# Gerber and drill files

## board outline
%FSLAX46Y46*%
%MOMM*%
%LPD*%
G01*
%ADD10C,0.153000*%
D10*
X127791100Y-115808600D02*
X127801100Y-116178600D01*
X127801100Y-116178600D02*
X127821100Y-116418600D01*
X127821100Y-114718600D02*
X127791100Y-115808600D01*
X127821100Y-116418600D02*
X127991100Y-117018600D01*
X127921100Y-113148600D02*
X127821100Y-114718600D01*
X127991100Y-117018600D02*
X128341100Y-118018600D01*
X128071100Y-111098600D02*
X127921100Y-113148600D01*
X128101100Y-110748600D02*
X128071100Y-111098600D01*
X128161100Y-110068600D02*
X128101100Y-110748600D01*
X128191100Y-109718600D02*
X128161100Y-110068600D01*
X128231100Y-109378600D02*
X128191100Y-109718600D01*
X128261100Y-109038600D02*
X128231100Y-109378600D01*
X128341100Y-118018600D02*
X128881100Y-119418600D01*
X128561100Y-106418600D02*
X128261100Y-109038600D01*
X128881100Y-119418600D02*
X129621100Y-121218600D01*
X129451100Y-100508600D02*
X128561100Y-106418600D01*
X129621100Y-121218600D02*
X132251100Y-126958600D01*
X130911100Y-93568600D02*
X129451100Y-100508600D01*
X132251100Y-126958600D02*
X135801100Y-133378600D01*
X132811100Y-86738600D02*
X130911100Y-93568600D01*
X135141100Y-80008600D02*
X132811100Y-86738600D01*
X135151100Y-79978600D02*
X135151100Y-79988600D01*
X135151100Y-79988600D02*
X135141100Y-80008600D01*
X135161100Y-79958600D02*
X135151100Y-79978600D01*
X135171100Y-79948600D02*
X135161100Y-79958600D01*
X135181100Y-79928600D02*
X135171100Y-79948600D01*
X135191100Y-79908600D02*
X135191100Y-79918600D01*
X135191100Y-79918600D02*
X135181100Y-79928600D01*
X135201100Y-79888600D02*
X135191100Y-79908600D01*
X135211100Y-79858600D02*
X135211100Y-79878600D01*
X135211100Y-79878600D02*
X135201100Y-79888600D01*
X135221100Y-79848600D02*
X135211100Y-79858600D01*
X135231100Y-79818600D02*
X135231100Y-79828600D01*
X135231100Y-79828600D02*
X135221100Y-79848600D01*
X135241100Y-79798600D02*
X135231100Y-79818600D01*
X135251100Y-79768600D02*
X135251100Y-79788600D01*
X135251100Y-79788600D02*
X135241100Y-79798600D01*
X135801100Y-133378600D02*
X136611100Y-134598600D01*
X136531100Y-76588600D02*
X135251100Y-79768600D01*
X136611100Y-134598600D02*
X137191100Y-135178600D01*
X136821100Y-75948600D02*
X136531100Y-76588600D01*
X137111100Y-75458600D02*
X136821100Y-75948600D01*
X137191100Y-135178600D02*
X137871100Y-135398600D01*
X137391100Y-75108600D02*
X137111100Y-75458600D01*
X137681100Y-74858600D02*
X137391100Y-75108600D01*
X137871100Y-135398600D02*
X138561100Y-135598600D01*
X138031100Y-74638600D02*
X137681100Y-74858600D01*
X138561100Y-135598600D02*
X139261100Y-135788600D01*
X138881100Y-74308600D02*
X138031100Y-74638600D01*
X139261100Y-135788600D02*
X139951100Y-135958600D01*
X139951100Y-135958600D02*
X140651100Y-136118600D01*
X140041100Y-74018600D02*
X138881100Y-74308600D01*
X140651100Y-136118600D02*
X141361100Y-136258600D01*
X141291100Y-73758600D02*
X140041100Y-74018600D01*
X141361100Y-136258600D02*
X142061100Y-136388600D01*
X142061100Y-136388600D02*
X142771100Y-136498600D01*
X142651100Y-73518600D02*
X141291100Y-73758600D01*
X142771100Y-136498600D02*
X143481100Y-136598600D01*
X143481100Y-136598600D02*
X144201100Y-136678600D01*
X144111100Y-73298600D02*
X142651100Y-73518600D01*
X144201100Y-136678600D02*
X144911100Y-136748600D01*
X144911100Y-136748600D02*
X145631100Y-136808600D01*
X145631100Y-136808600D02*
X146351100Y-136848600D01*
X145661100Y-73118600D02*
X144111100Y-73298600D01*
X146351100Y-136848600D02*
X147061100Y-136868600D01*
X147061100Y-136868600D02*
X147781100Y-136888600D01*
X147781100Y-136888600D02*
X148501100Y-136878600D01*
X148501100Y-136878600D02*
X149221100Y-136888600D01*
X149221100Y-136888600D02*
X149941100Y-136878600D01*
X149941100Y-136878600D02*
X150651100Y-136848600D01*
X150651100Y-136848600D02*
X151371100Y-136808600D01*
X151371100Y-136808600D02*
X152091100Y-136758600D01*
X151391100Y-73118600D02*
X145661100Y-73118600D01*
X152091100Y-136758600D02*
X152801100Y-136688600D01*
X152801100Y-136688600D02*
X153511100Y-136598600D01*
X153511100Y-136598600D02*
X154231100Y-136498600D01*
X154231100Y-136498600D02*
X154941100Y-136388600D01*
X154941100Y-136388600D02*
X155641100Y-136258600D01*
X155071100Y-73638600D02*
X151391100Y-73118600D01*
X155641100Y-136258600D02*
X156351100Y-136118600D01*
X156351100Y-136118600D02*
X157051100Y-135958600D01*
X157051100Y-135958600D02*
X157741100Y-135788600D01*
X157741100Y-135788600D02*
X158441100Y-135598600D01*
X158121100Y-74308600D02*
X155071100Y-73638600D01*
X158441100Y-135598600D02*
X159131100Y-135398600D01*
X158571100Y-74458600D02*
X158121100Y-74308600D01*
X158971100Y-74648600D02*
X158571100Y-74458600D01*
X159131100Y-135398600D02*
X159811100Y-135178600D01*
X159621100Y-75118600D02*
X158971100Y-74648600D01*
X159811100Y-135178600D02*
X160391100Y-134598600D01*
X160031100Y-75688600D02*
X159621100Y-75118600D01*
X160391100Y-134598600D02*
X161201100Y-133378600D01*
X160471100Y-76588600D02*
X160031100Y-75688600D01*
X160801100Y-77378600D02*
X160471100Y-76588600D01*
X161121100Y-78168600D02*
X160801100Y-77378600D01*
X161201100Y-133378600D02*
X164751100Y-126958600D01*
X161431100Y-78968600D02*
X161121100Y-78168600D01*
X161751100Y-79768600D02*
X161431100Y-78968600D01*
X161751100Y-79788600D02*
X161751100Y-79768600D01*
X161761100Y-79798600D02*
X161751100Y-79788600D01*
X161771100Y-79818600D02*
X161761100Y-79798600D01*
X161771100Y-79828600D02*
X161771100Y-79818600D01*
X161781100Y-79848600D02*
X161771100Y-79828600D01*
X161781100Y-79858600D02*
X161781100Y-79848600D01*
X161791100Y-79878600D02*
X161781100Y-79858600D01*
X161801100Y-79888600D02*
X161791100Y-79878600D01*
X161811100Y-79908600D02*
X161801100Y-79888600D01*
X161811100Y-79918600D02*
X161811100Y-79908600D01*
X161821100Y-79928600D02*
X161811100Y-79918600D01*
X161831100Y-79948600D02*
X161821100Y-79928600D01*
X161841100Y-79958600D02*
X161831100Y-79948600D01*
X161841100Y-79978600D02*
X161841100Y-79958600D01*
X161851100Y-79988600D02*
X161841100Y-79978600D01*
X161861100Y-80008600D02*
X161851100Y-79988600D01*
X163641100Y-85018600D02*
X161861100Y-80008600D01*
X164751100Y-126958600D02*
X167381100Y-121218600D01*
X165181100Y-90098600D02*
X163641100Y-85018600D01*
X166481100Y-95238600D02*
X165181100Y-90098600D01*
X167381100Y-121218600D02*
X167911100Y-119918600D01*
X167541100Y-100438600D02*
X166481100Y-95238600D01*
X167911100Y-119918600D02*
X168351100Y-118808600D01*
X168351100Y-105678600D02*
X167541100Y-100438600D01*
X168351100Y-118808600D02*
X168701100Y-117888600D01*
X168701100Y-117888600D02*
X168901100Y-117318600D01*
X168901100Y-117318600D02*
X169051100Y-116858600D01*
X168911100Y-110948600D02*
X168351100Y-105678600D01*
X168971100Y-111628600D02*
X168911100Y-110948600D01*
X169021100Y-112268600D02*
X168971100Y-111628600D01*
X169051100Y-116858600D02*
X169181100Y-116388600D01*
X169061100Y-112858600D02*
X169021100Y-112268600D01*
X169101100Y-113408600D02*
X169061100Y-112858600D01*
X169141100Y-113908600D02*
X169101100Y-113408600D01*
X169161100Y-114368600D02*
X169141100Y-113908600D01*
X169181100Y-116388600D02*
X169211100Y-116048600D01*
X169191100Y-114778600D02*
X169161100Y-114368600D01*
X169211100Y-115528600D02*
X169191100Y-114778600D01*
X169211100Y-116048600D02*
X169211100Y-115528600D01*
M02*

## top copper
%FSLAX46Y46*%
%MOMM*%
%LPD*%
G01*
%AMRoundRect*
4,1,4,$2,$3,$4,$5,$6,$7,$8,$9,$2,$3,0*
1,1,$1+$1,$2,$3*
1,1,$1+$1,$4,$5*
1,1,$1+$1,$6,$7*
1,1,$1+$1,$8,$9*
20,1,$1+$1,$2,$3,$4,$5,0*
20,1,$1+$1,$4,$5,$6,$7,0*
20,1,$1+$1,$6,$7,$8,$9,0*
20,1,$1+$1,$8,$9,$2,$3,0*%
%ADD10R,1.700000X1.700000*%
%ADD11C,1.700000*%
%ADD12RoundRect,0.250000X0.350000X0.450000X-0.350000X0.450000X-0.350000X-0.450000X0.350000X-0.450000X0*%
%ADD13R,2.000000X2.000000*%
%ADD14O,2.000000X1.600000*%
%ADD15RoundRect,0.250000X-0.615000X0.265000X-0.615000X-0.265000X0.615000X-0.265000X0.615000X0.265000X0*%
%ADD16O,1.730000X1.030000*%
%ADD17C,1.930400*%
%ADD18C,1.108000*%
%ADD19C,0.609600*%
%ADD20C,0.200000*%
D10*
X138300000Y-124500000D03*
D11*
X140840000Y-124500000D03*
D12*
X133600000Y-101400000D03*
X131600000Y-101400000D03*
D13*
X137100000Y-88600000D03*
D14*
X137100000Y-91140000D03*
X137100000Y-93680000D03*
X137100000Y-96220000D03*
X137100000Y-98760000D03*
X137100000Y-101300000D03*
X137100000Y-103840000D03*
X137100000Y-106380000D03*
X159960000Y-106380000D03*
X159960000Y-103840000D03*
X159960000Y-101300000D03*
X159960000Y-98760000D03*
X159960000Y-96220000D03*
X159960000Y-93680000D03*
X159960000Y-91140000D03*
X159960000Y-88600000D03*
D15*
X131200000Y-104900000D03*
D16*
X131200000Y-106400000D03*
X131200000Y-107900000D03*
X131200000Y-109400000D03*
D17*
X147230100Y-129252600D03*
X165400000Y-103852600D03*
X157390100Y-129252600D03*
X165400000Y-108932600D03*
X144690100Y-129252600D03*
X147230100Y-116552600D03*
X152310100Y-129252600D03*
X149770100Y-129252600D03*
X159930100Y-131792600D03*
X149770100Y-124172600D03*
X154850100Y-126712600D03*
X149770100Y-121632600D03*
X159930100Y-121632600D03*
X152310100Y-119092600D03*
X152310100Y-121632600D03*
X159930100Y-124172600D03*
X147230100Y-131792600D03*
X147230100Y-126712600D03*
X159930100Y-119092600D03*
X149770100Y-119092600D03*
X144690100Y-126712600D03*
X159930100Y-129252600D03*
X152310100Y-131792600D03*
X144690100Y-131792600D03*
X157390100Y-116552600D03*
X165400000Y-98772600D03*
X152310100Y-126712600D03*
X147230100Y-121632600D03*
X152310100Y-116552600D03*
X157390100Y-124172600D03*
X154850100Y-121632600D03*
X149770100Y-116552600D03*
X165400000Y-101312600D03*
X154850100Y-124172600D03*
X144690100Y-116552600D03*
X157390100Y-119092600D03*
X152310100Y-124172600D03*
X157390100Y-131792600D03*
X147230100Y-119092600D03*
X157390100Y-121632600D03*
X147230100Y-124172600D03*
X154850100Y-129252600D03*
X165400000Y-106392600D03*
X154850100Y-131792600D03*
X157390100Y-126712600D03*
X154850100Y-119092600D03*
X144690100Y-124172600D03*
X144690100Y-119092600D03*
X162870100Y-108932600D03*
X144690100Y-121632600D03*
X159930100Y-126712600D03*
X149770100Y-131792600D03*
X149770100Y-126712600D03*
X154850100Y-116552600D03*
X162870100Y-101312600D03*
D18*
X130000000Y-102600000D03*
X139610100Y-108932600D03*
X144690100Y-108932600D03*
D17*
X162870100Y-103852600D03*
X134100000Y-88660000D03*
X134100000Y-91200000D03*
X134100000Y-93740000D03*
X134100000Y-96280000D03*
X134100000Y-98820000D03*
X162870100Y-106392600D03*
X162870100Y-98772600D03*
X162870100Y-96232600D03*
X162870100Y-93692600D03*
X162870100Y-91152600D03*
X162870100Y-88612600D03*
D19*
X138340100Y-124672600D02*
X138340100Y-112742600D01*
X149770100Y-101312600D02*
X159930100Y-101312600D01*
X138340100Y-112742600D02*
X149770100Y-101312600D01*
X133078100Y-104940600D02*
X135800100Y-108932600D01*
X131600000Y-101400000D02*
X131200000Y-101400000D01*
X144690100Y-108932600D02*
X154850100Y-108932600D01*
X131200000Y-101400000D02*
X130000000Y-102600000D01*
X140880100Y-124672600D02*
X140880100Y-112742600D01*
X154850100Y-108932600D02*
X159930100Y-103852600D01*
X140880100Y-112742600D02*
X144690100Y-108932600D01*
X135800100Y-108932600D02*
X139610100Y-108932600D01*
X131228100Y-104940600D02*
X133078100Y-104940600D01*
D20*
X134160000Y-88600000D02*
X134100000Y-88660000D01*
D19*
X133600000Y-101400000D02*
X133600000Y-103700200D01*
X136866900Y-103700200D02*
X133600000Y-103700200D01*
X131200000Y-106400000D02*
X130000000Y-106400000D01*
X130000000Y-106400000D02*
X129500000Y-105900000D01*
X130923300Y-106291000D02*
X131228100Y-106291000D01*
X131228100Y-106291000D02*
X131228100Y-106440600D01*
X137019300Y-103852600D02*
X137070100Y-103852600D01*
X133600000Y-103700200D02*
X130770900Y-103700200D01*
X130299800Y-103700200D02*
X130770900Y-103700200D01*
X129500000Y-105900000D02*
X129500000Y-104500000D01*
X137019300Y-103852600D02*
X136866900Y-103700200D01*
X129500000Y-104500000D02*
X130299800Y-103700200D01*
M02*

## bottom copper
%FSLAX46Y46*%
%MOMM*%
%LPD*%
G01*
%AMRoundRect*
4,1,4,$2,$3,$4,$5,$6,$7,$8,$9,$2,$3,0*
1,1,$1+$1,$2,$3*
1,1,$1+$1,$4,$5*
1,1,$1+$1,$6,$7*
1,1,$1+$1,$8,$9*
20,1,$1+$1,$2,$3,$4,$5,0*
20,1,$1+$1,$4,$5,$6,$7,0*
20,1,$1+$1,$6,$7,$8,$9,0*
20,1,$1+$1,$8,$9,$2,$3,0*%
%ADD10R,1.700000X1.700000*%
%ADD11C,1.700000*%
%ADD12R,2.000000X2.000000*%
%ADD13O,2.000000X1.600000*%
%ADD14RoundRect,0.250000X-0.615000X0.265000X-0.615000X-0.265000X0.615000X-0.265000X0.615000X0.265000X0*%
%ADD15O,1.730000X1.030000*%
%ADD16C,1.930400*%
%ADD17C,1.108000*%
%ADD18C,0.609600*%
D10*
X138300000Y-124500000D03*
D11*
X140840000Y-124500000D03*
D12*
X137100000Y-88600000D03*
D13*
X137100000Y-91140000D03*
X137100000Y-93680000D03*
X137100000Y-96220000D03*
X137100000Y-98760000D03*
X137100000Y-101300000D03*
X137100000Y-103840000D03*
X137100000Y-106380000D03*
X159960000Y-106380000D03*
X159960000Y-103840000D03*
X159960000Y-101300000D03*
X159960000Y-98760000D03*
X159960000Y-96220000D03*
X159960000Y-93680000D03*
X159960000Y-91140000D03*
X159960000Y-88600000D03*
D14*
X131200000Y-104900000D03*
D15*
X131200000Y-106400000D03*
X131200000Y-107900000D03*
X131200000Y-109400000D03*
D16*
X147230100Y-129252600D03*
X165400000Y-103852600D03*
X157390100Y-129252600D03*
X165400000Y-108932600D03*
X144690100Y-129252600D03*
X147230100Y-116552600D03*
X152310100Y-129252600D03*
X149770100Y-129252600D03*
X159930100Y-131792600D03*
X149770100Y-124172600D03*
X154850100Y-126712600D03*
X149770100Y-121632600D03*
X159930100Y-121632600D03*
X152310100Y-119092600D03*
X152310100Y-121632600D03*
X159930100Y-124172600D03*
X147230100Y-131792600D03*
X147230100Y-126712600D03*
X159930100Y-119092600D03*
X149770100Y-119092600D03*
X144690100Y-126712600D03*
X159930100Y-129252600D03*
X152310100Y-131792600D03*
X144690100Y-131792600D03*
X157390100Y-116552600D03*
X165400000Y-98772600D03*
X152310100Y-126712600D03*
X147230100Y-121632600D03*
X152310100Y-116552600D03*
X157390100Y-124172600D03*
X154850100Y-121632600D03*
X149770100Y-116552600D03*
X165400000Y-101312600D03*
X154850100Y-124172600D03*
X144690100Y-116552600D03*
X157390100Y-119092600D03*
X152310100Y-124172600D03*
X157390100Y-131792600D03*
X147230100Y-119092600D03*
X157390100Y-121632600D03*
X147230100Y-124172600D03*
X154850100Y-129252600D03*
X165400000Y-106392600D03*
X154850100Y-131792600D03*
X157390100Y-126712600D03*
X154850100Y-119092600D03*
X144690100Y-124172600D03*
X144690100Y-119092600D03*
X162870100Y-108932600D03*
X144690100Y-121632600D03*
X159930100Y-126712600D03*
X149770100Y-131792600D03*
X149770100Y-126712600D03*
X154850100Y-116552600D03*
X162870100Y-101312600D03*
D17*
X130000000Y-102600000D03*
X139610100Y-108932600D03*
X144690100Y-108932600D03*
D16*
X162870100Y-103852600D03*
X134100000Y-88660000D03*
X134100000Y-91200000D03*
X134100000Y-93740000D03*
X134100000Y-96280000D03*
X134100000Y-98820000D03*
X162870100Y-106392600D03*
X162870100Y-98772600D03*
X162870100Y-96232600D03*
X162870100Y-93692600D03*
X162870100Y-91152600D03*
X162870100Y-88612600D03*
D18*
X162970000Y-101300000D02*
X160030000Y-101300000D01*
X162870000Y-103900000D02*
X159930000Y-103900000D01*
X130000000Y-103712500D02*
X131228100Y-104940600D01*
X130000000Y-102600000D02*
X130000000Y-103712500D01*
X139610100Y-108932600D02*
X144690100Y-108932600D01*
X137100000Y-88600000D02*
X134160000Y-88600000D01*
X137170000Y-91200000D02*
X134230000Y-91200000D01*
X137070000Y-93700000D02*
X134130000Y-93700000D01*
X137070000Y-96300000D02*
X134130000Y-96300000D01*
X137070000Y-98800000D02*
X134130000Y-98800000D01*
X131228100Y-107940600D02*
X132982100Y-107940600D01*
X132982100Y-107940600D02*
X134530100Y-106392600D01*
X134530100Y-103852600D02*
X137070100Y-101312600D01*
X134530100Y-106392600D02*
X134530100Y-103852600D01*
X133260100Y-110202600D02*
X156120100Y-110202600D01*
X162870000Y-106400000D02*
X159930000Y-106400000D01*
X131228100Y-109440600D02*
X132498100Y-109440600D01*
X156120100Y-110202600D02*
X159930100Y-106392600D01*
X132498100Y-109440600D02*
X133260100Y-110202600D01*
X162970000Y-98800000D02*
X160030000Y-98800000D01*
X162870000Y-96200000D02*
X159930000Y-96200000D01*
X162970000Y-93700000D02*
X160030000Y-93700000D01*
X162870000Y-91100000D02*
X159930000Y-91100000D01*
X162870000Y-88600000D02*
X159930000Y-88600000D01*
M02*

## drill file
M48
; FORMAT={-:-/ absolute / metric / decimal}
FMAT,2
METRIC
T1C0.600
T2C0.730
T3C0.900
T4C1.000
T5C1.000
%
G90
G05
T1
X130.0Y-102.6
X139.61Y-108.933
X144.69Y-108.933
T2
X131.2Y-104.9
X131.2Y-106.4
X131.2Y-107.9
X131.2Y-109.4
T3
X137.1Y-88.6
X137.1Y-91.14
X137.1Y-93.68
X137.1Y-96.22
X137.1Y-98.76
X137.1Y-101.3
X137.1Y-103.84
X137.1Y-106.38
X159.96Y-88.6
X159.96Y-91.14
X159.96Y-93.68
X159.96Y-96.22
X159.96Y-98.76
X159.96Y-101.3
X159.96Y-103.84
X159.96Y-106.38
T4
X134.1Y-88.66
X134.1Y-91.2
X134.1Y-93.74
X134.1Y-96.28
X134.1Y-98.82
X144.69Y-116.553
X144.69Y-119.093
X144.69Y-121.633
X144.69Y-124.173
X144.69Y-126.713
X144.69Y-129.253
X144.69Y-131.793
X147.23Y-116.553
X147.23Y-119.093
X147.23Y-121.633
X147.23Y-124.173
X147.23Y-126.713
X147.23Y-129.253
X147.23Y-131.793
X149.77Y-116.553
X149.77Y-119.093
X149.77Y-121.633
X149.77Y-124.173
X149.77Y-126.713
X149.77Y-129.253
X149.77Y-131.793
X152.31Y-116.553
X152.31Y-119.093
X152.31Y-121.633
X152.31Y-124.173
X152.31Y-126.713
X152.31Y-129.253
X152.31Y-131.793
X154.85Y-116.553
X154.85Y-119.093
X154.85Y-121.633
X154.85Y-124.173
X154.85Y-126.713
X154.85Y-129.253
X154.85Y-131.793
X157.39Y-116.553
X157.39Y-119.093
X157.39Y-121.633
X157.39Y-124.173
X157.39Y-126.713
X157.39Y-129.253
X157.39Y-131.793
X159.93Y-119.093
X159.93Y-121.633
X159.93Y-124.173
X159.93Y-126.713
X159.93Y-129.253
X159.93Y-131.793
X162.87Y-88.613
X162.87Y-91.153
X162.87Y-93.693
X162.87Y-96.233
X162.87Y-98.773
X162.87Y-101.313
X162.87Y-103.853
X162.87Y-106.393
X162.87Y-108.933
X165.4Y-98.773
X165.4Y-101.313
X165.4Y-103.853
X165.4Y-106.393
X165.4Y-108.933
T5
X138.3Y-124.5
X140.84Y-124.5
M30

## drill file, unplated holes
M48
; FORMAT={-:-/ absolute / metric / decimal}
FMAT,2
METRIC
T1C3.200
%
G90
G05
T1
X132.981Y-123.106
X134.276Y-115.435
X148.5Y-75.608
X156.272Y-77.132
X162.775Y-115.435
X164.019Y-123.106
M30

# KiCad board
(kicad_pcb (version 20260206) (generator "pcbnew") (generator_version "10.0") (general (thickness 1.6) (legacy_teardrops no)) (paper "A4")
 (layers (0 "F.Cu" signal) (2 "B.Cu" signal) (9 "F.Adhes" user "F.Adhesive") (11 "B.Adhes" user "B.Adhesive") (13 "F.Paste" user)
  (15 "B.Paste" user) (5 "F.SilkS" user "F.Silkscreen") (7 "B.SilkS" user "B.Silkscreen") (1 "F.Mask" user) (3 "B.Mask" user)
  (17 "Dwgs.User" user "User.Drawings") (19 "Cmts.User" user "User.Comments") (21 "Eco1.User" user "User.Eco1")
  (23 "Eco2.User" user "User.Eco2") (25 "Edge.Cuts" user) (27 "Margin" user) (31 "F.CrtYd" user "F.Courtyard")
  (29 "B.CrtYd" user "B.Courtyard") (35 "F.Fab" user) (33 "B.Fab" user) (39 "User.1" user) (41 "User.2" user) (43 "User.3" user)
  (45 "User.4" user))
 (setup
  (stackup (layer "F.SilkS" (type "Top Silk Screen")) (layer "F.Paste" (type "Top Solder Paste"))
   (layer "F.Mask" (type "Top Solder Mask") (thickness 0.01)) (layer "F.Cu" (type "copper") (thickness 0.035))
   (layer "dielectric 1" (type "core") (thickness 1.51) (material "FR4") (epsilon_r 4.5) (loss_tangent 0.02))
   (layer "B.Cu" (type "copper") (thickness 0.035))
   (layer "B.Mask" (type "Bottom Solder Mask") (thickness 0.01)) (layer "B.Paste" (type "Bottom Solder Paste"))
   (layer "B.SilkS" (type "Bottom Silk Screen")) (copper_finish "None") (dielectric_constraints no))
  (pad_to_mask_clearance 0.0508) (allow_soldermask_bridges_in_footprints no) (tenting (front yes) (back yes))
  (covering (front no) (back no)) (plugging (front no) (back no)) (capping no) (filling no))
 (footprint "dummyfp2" (layer "F.Cu") (at 162.7749 115.435)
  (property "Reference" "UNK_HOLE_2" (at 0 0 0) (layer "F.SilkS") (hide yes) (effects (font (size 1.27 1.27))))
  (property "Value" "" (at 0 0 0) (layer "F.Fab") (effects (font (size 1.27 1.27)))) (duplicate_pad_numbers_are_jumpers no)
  (pad "" np_thru_hole circle (at 0 0) (size 3.2 3.2) (drill 3.2) (layers "*.Cu" "*.Mask")))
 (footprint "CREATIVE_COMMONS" (layer "F.Cu") (at 112.9401 148.3026)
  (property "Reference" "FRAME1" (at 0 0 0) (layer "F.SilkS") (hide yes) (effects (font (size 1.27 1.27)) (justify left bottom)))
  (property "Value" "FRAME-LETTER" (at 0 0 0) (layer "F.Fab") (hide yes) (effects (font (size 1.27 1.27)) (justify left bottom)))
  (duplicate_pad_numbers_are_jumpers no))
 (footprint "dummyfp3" (layer "F.Cu") (at 132.9807 123.1058)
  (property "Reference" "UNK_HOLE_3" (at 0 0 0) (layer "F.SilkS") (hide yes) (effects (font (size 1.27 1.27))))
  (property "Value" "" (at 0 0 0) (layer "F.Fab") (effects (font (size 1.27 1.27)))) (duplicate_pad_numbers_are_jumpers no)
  (pad "" np_thru_hole circle (at 0 0) (size 3.2 3.2) (drill 3.2) (layers "*.Cu" "*.Mask")))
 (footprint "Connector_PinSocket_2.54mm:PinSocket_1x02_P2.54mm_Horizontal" (layer "F.Cu") (at 138.3 124.5 90)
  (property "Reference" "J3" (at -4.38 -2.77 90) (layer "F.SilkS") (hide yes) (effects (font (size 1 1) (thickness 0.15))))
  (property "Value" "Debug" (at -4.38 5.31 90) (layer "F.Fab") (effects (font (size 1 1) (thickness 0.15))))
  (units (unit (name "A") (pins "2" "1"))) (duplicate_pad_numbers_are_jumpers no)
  (pad "1" thru_hole rect (at 0 0 90) (size 1.7 1.7) (drill 1) (layers "*.Cu" "*.Mask") (remove_unused_layers no) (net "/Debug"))
  (pad "2" thru_hole circle (at 0 2.54 90) (size 1.7 1.7) (drill 1) (layers "*.Cu" "*.Mask") (remove_unused_layers no) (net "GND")))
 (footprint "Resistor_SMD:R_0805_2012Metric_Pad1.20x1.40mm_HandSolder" (layer "F.Cu") (at 132.6 101.4 180)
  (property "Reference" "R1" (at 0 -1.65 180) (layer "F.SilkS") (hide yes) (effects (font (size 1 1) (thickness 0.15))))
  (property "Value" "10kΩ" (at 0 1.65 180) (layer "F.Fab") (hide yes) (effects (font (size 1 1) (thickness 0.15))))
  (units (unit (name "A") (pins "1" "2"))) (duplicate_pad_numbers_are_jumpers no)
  (pad "1" smd roundrect (at -1 0 180) (size 1.2 1.4) (layers "F.Cu" "F.Mask" "F.Paste") (roundrect_rratio 0.208333) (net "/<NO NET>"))
  (pad "2" smd roundrect (at 1 0 180) (size 1.2 1.4) (layers "F.Cu" "F.Mask" "F.Paste") (roundrect_rratio 0.208333) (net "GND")))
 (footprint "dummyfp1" (layer "F.Cu") (at 156.2725 77.1318)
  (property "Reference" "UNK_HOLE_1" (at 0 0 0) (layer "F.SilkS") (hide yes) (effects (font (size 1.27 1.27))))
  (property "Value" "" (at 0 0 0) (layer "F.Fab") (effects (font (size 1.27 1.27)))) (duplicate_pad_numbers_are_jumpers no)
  (pad "" np_thru_hole circle (at 0 0) (size 3.2 3.2) (drill 3.2) (layers "*.Cu" "*.Mask")))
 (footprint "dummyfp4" (layer "F.Cu") (at 164.0195 123.1058)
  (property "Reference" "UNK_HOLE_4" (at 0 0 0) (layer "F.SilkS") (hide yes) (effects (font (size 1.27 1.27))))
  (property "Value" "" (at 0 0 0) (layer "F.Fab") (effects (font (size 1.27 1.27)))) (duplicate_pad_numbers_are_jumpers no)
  (pad "" np_thru_hole circle (at 0 0) (size 3.2 3.2) (drill 3.2) (layers "*.Cu" "*.Mask")))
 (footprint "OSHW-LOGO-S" (layer "F.Cu") (at 142.2 77.2)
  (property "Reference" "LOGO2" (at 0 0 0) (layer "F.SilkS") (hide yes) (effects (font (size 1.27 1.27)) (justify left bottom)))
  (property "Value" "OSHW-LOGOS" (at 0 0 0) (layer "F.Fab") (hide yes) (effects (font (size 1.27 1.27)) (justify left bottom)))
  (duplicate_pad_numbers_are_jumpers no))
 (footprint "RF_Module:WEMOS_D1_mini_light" (layer "F.Cu") (at 137.1 88.6)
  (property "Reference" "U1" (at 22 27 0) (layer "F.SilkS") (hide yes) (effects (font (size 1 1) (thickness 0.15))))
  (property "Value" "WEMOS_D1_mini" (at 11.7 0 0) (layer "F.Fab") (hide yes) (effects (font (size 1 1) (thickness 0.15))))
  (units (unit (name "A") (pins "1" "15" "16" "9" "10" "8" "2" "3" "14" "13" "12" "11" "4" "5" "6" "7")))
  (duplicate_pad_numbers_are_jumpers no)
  (pad "1" thru_hole rect (at 0 0) (size 2 2) (drill 0.9) (layers "*.Cu" "*.Mask") (remove_unused_layers no)
   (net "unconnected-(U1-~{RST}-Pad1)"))
  (pad "2" thru_hole oval (at 0 2.54) (size 2 1.6) (drill 0.9) (layers "*.Cu" "*.Mask") (remove_unused_layers no)
   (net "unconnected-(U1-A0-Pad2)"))
  (pad "3" thru_hole oval (at 0 5.08) (size 2 1.6) (drill 0.9) (layers "*.Cu" "*.Mask") (remove_unused_layers no)
   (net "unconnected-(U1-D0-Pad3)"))
  (pad "4" thru_hole oval (at 0 7.62) (size 2 1.6) (drill 0.9) (layers "*.Cu" "*.Mask") (remove_unused_layers no)
   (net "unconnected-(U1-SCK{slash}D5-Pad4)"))
  (pad "5" thru_hole oval (at 0 10.16) (size 2 1.6) (drill 0.9) (layers "*.Cu" "*.Mask") (remove_unused_layers no)
   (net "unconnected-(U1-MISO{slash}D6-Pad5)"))
  (pad "6" thru_hole oval (at 0 12.7) (size 2 1.6) (drill 0.9) (layers "*.Cu" "*.Mask") (remove_unused_layers no) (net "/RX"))
  (pad "7" thru_hole oval (at 0 15.24) (size 2 1.6) (drill 0.9) (layers "*.Cu" "*.Mask") (remove_unused_layers no) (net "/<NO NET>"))
  (pad "8" thru_hole oval (at 0 17.78) (size 2 1.6) (drill 0.9) (layers "*.Cu" "*.Mask") (remove_unused_layers no)
   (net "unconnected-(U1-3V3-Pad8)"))
  (pad "9" thru_hole oval (at 22.86 17.78) (size 2 1.6) (drill 0.9) (layers "*.Cu" "*.Mask") (remove_unused_layers no) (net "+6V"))
  (pad "10" thru_hole oval (at 22.86 15.24) (size 2 1.6) (drill 0.9) (layers "*.Cu" "*.Mask") (remove_unused_layers no) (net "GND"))
  (pad "11" thru_hole oval (at 22.86 12.7) (size 2 1.6) (drill 0.9) (layers "*.Cu" "*.Mask") (remove_unused_layers no) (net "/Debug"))
  (pad "12" thru_hole oval (at 22.86 10.16) (size 2 1.6) (drill 0.9) (layers "*.Cu" "*.Mask") (remove_unused_layers no)
   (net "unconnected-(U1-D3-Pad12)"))
  (pad "13" thru_hole oval (at 22.86 7.62) (size 2 1.6) (drill 0.9) (layers "*.Cu" "*.Mask") (remove_unused_layers no)
   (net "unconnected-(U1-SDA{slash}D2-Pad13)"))
  (pad "14" thru_hole oval (at 22.86 5.08) (size 2 1.6) (drill 0.9) (layers "*.Cu" "*.Mask") (remove_unused_layers no)
   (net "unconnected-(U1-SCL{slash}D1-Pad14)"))
  (pad "15" thru_hole oval (at 22.86 2.54) (size 2 1.6) (drill 0.9) (layers "*.Cu" "*.Mask") (remove_unused_layers no)
   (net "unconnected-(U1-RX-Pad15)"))
  (pad "16" thru_hole oval (at 22.86 0) (size 2 1.6) (drill 0.9) (layers "*.Cu" "*.Mask") (remove_unused_layers no)
   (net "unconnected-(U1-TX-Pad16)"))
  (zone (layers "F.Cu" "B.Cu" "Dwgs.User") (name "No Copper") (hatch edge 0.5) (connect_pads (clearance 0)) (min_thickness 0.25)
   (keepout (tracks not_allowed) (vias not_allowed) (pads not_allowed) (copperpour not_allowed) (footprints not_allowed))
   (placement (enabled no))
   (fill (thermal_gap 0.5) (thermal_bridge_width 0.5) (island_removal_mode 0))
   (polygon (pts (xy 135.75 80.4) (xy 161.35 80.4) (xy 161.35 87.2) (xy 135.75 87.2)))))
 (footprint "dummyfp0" (layer "F.Cu") (at 148.5001 75.6078)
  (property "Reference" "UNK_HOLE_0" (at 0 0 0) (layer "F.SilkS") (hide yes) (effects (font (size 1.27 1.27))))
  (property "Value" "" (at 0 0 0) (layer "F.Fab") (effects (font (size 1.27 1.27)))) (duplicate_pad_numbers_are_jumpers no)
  (pad "" np_thru_hole circle (at 0 0) (size 3.2 3.2) (drill 3.2) (layers "*.Cu" "*.Mask")))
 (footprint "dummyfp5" (layer "F.Cu") (at 134.2761 115.435)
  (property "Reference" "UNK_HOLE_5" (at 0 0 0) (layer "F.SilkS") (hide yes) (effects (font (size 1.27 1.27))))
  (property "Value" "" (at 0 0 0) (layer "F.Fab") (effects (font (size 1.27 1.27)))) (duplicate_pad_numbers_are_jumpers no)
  (pad "" np_thru_hole circle (at 0 0) (size 3.2 3.2) (drill 3.2) (layers "*.Cu" "*.Mask")))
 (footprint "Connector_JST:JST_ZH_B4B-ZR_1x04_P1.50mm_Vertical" (layer "B.Cu") (at 131.2 104.9 -90)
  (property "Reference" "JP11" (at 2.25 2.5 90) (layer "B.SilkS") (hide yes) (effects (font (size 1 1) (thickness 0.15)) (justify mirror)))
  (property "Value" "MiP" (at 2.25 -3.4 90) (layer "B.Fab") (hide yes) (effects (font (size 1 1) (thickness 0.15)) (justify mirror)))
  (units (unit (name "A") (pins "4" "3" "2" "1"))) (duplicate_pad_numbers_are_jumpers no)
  (pad "1" thru_hole roundrect (at 0 0 270) (size 1.03 1.73) (drill 0.73) (layers "*.Cu" "*.Mask") (remove_unused_layers no)
   (roundrect_rratio 0.242718) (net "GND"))
  (pad "2" thru_hole oval (at 1.5 0 270) (size 1.03 1.73) (drill 0.73) (layers "*.Cu" "*.Mask") (remove_unused_layers no) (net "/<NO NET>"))
  (pad "3" thru_hole oval (at 3 0 270) (size 1.03 1.73) (drill 0.73) (layers "*.Cu" "*.Mask") (remove_unused_layers no) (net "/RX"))
  (pad "4" thru_hole oval (at 4.5 0 270) (size 1.03 1.73) (drill 0.73) (layers "*.Cu" "*.Mask") (remove_unused_layers no) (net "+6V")))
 (gr_line (start 127.7911 115.8086) (end 127.8011 116.1786) (stroke (width 0.153) (type solid)) (layer "Edge.Cuts"))
 (gr_line (start 127.8011 116.1786) (end 127.8211 116.4186) (stroke (width 0.153) (type solid)) (layer "Edge.Cuts"))
 (gr_line (start 127.8211 114.7186) (end 127.7911 115.8086) (stroke (width 0.153) (type solid)) (layer "Edge.Cuts"))
 (gr_line (start 127.8211 116.4186) (end 127.9911 117.0186) (stroke (width 0.153) (type solid)) (layer "Edge.Cuts"))
 (gr_line (start 127.9211 113.1486) (end 127.8211 114.7186) (stroke (width 0.153) (type solid)) (layer "Edge.Cuts"))
 (gr_line (start 127.9911 117.0186) (end 128.3411 118.0186) (stroke (width 0.153) (type solid)) (layer "Edge.Cuts"))
 (gr_line (start 128.0711 111.0986) (end 127.9211 113.1486) (stroke (width 0.153) (type solid)) (layer "Edge.Cuts"))
 (gr_line (start 128.1011 110.7486) (end 128.0711 111.0986) (stroke (width 0.153) (type solid)) (layer "Edge.Cuts"))
 (gr_line (start 128.1611 110.0686) (end 128.1011 110.7486) (stroke (width 0.153) (type solid)) (layer "Edge.Cuts"))
 (gr_line (start 128.1911 109.7186) (end 128.1611 110.0686) (stroke (width 0.153) (type solid)) (layer "Edge.Cuts"))
 (gr_line (start 128.2311 109.3786) (end 128.1911 109.7186) (stroke (width 0.153) (type solid)) (layer "Edge.Cuts"))
 (gr_line (start 128.2611 109.0386) (end 128.2311 109.3786) (stroke (width 0.153) (type solid)) (layer "Edge.Cuts"))
 (gr_line (start 128.3411 118.0186) (end 128.8811 119.4186) (stroke (width 0.153) (type solid)) (layer "Edge.Cuts"))
 (gr_line (start 128.5611 106.4186) (end 128.2611 109.0386) (stroke (width 0.153) (type solid)) (layer "Edge.Cuts"))
 (gr_line (start 128.8811 119.4186) (end 129.6211 121.2186) (stroke (width 0.153) (type solid)) (layer "Edge.Cuts"))
 (gr_line (start 129.4511 100.5086) (end 128.5611 106.4186) (stroke (width 0.153) (type solid)) (layer "Edge.Cuts"))
 (gr_line (start 129.6211 121.2186) (end 132.2511 126.9586) (stroke (width 0.153) (type solid)) (layer "Edge.Cuts"))
 (gr_line (start 130.9111 93.5686) (end 129.4511 100.5086) (stroke (width 0.153) (type solid)) (layer "Edge.Cuts"))
 (gr_line (start 132.2511 126.9586) (end 135.8011 133.3786) (stroke (width 0.153) (type solid)) (layer "Edge.Cuts"))
 (gr_line (start 132.8111 86.7386) (end 130.9111 93.5686) (stroke (width 0.153) (type solid)) (layer "Edge.Cuts"))
 (gr_line (start 135.1411 80.0086) (end 132.8111 86.7386) (stroke (width 0.153) (type solid)) (layer "Edge.Cuts"))
 (gr_line (start 135.1511 79.9786) (end 135.1511 79.9886) (stroke (width 0.153) (type solid)) (layer "Edge.Cuts"))
 (gr_line (start 135.1511 79.9886) (end 135.1411 80.0086) (stroke (width 0.153) (type solid)) (layer "Edge.Cuts"))
 (gr_line (start 135.1611 79.9586) (end 135.1511 79.9786) (stroke (width 0.153) (type solid)) (layer "Edge.Cuts"))
 (gr_line (start 135.1711 79.9486) (end 135.1611 79.9586) (stroke (width 0.153) (type solid)) (layer "Edge.Cuts"))
 (gr_line (start 135.1811 79.9286) (end 135.1711 79.9486) (stroke (width 0.153) (type solid)) (layer "Edge.Cuts"))
 (gr_line (start 135.1911 79.9086) (end 135.1911 79.9186) (stroke (width 0.153) (type solid)) (layer "Edge.Cuts"))
 (gr_line (start 135.1911 79.9186) (end 135.1811 79.9286) (stroke (width 0.153) (type solid)) (layer "Edge.Cuts"))
 (gr_line (start 135.2011 79.8886) (end 135.1911 79.9086) (stroke (width 0.153) (type solid)) (layer "Edge.Cuts"))
 (gr_line (start 135.2111 79.8586) (end 135.2111 79.8786) (stroke (width 0.153) (type solid)) (layer "Edge.Cuts"))
 (gr_line (start 135.2111 79.8786) (end 135.2011 79.8886) (stroke (width 0.153) (type solid)) (layer "Edge.Cuts"))
 (gr_line (start 135.2211 79.8486) (end 135.2111 79.8586) (stroke (width 0.153) (type solid)) (layer "Edge.Cuts"))
 (gr_line (start 135.2311 79.8186) (end 135.2311 79.8286) (stroke (width 0.153) (type solid)) (layer "Edge.Cuts"))
 (gr_line (start 135.2311 79.8286) (end 135.2211 79.8486) (stroke (width 0.153) (type solid)) (layer "Edge.Cuts"))
 (gr_line (start 135.2411 79.7986) (end 135.2311 79.8186) (stroke (width 0.153) (type solid)) (layer "Edge.Cuts"))
 (gr_line (start 135.2511 79.7686) (end 135.2511 79.7886) (stroke (width 0.153) (type solid)) (layer "Edge.Cuts"))
 (gr_line (start 135.2511 79.7886) (end 135.2411 79.7986) (stroke (width 0.153) (type solid)) (layer "Edge.Cuts"))
 (gr_line (start 135.8011 133.3786) (end 136.6111 134.5986) (stroke (width 0.153) (type solid)) (layer "Edge.Cuts"))
 (gr_line (start 136.5311 76.5886) (end 135.2511 79.7686) (stroke (width 0.153) (type solid)) (layer "Edge.Cuts"))
 (gr_line (start 136.6111 134.5986) (end 137.1911 135.1786) (stroke (width 0.153) (type solid)) (layer "Edge.Cuts"))
 (gr_line (start 136.8211 75.9486) (end 136.5311 76.5886) (stroke (width 0.153) (type solid)) (layer "Edge.Cuts"))
 (gr_line (start 137.1111 75.4586) (end 136.8211 75.9486) (stroke (width 0.153) (type solid)) (layer "Edge.Cuts"))
 (gr_line (start 137.1911 135.1786) (end 137.8711 135.3986) (stroke (width 0.153) (type solid)) (layer "Edge.Cuts"))
 (gr_line (start 137.3911 75.1086) (end 137.1111 75.4586) (stroke (width 0.153) (type solid)) (layer "Edge.Cuts"))
 (gr_line (start 137.6811 74.8586) (end 137.3911 75.1086) (stroke (width 0.153) (type solid)) (layer "Edge.Cuts"))
 (gr_line (start 137.8711 135.3986) (end 138.5611 135.5986) (stroke (width 0.153) (type solid)) (layer "Edge.Cuts"))
 (gr_line (start 138.0311 74.6386) (end 137.6811 74.8586) (stroke (width 0.153) (type solid)) (layer "Edge.Cuts"))
 (gr_line (start 138.5611 135.5986) (end 139.2611 135.7886) (stroke (width 0.153) (type solid)) (layer "Edge.Cuts"))
 (gr_line (start 138.8811 74.3086) (end 138.0311 74.6386) (stroke (width 0.153) (type solid)) (layer "Edge.Cuts"))
 (gr_line (start 139.2611 135.7886) (end 139.9511 135.9586) (stroke (width 0.153) (type solid)) (layer "Edge.Cuts"))
 (gr_line (start 139.9511 135.9586) (end 140.6511 136.1186) (stroke (width 0.153) (type solid)) (layer "Edge.Cuts"))
 (gr_line (start 140.0411 74.0186) (end 138.8811 74.3086) (stroke (width 0.153) (type solid)) (layer "Edge.Cuts"))
 (gr_line (start 140.6511 136.1186) (end 141.3611 136.2586) (stroke (width 0.153) (type solid)) (layer "Edge.Cuts"))
 (gr_line (start 141.2911 73.7586) (end 140.0411 74.0186) (stroke (width 0.153) (type solid)) (layer "Edge.Cuts"))
 (gr_line (start 141.3611 136.2586) (end 142.0611 136.3886) (stroke (width 0.153) (type solid)) (layer "Edge.Cuts"))
 (gr_line (start 142.0611 136.3886) (end 142.7711 136.4986) (stroke (width 0.153) (type solid)) (layer "Edge.Cuts"))
 (gr_line (start 142.6511 73.5186) (end 141.2911 73.7586) (stroke (width 0.153) (type solid)) (layer "Edge.Cuts"))
 (gr_line (start 142.7711 136.4986) (end 143.4811 136.5986) (stroke (width 0.153) (type solid)) (layer "Edge.Cuts"))
 (gr_line (start 143.4811 136.5986) (end 144.2011 136.6786) (stroke (width 0.153) (type solid)) (layer "Edge.Cuts"))
 (gr_line (start 144.1111 73.2986) (end 142.6511 73.5186) (stroke (width 0.153) (type solid)) (layer "Edge.Cuts"))
 (gr_line (start 144.2011 136.6786) (end 144.9111 136.7486) (stroke (width 0.153) (type solid)) (layer "Edge.Cuts"))
 (gr_line (start 144.9111 136.7486) (end 145.6311 136.8086) (stroke (width 0.153) (type solid)) (layer "Edge.Cuts"))
 (gr_line (start 145.6311 136.8086) (end 146.3511 136.8486) (stroke (width 0.153) (type solid)) (layer "Edge.Cuts"))
 (gr_line (start 145.6611 73.1186) (end 144.1111 73.2986) (stroke (width 0.153) (type solid)) (layer "Edge.Cuts"))
 (gr_line (start 146.3511 136.8486) (end 147.0611 136.8686) (stroke (width 0.153) (type solid)) (layer "Edge.Cuts"))
 (gr_line (start 147.0611 136.8686) (end 147.7811 136.8886) (stroke (width 0.153) (type solid)) (layer "Edge.Cuts"))
 (gr_line (start 147.7811 136.8886) (end 148.5011 136.8786) (stroke (width 0.153) (type solid)) (layer "Edge.Cuts"))
 (gr_line (start 148.5011 136.8786) (end 149.2211 136.8886) (stroke (width 0.153) (type solid)) (layer "Edge.Cuts"))
 (gr_line (start 149.2211 136.8886) (end 149.9411 136.8786) (stroke (width 0.153) (type solid)) (layer "Edge.Cuts"))
 (gr_line (start 149.9411 136.8786) (end 150.6511 136.8486) (stroke (width 0.153) (type solid)) (layer "Edge.Cuts"))
 (gr_line (start 150.6511 136.8486) (end 151.3711 136.8086) (stroke (width 0.153) (type solid)) (layer "Edge.Cuts"))
 (gr_line (start 151.3711 136.8086) (end 152.0911 136.7586) (stroke (width 0.153) (type solid)) (layer "Edge.Cuts"))
 (gr_line (start 151.3911 73.1186) (end 145.6611 73.1186) (stroke (width 0.153) (type solid)) (layer "Edge.Cuts"))
 (gr_line (start 152.0911 136.7586) (end 152.8011 136.6886) (stroke (width 0.153) (type solid)) (layer "Edge.Cuts"))
 (gr_line (start 152.8011 136.6886) (end 153.5111 136.5986) (stroke (width 0.153) (type solid)) (layer "Edge.Cuts"))
 (gr_line (start 153.5111 136.5986) (end 154.2311 136.4986) (stroke (width 0.153) (type solid)) (layer "Edge.Cuts"))
 (gr_line (start 154.2311 136.4986) (end 154.9411 136.3886) (stroke (width 0.153) (type solid)) (layer "Edge.Cuts"))
 (gr_line (start 154.9411 136.3886) (end 155.6411 136.2586) (stroke (width 0.153) (type solid)) (layer "Edge.Cuts"))
 (gr_line (start 155.0711 73.6386) (end 151.3911 73.1186) (stroke (width 0.153) (type solid)) (layer "Edge.Cuts"))
 (gr_line (start 155.6411 136.2586) (end 156.3511 136.1186) (stroke (width 0.153) (type solid)) (layer "Edge.Cuts"))
 (gr_line (start 156.3511 136.1186) (end 157.0511 135.9586) (stroke (width 0.153) (type solid)) (layer "Edge.Cuts"))
 (gr_line (start 157.0511 135.9586) (end 157.7411 135.7886) (stroke (width 0.153) (type solid)) (layer "Edge.Cuts"))
 (gr_line (start 157.7411 135.7886) (end 158.4411 135.5986) (stroke (width 0.153) (type solid)) (layer "Edge.Cuts"))
 (gr_line (start 158.1211 74.3086) (end 155.0711 73.6386) (stroke (width 0.153) (type solid)) (layer "Edge.Cuts"))
 (gr_line (start 158.4411 135.5986) (end 159.1311 135.3986) (stroke (width 0.153) (type solid)) (layer "Edge.Cuts"))
 (gr_line (start 158.5711 74.4586) (end 158.1211 74.3086) (stroke (width 0.153) (type solid)) (layer "Edge.Cuts"))
 (gr_line (start 158.9711 74.6486) (end 158.5711 74.4586) (stroke (width 0.153) (type solid)) (layer "Edge.Cuts"))
 (gr_line (start 159.1311 135.3986) (end 159.8111 135.1786) (stroke (width 0.153) (type solid)) (layer "Edge.Cuts"))
 (gr_line (start 159.6211 75.1186) (end 158.9711 74.6486) (stroke (width 0.153) (type solid)) (layer "Edge.Cuts"))
 (gr_line (start 159.8111 135.1786) (end 160.3911 134.5986) (stroke (width 0.153) (type solid)) (layer "Edge.Cuts"))
 (gr_line (start 160.0311 75.6886) (end 159.6211 75.1186) (stroke (width 0.153) (type solid)) (layer "Edge.Cuts"))
 (gr_line (start 160.3911 134.5986) (end 161.2011 133.3786) (stroke (width 0.153) (type solid)) (layer "Edge.Cuts"))
 (gr_line (start 160.4711 76.5886) (end 160.0311 75.6886) (stroke (width 0.153) (type solid)) (layer "Edge.Cuts"))
 (gr_line (start 160.8011 77.3786) (end 160.4711 76.5886) (stroke (width 0.153) (type solid)) (layer "Edge.Cuts"))
 (gr_line (start 161.1211 78.1686) (end 160.8011 77.3786) (stroke (width 0.153) (type solid)) (layer "Edge.Cuts"))
 (gr_line (start 161.2011 133.3786) (end 164.7511 126.9586) (stroke (width 0.153) (type solid)) (layer "Edge.Cuts"))
 (gr_line (start 161.4311 78.9686) (end 161.1211 78.1686) (stroke (width 0.153) (type solid)) (layer "Edge.Cuts"))
 (gr_line (start 161.7511 79.7686) (end 161.4311 78.9686) (stroke (width 0.153) (type solid)) (layer "Edge.Cuts"))
 (gr_line (start 161.7511 79.7886) (end 161.7511 79.7686) (stroke (width 0.153) (type solid)) (layer "Edge.Cuts"))
 (gr_line (start 161.7611 79.7986) (end 161.7511 79.7886) (stroke (width 0.153) (type solid)) (layer "Edge.Cuts"))
 (gr_line (start 161.7711 79.8186) (end 161.7611 79.7986) (stroke (width 0.153) (type solid)) (layer "Edge.Cuts"))
 (gr_line (start 161.7711 79.8286) (end 161.7711 79.8186) (stroke (width 0.153) (type solid)) (layer "Edge.Cuts"))
 (gr_line (start 161.7811 79.8486) (end 161.7711 79.8286) (stroke (width 0.153) (type solid)) (layer "Edge.Cuts"))
 (gr_line (start 161.7811 79.8586) (end 161.7811 79.8486) (stroke (width 0.153) (type solid)) (layer "Edge.Cuts"))
 (gr_line (start 161.7911 79.8786) (end 161.7811 79.8586) (stroke (width 0.153) (type solid)) (layer "Edge.Cuts"))
 (gr_line (start 161.8011 79.8886) (end 161.7911 79.8786) (stroke (width 0.153) (type solid)) (layer "Edge.Cuts"))
 (gr_line (start 161.8111 79.9086) (end 161.8011 79.8886) (stroke (width 0.153) (type solid)) (layer "Edge.Cuts"))
 (gr_line (start 161.8111 79.9186) (end 161.8111 79.9086) (stroke (width 0.153) (type solid)) (layer "Edge.Cuts"))
 (gr_line (start 161.8211 79.9286) (end 161.8111 79.9186) (stroke (width 0.153) (type solid)) (layer "Edge.Cuts"))
 (gr_line (start 161.8311 79.9486) (end 161.8211 79.9286) (stroke (width 0.153) (type solid)) (layer "Edge.Cuts"))
 (gr_line (start 161.8411 79.9586) (end 161.8311 79.9486) (stroke (width 0.153) (type solid)) (layer "Edge.Cuts"))
 (gr_line (start 161.8411 79.9786) (end 161.8411 79.9586) (stroke (width 0.153) (type solid)) (layer "Edge.Cuts"))
 (gr_line (start 161.8511 79.9886) (end 161.8411 79.9786) (stroke (width 0.153) (type solid)) (layer "Edge.Cuts"))
 (gr_line (start 161.8611 80.0086) (end 161.8511 79.9886) (stroke (width 0.153) (type solid)) (layer "Edge.Cuts"))
 (gr_line (start 163.6411 85.0186) (end 161.8611 80.0086) (stroke (width 0.153) (type solid)) (layer "Edge.Cuts"))
 (gr_line (start 164.7511 126.9586) (end 167.3811 121.2186) (stroke (width 0.153) (type solid)) (layer "Edge.Cuts"))
 (gr_line (start 165.1811 90.0986) (end 163.6411 85.0186) (stroke (width 0.153) (type solid)) (layer "Edge.Cuts"))
 (gr_line (start 166.4811 95.2386) (end 165.1811 90.0986) (stroke (width 0.153) (type solid)) (layer "Edge.Cuts"))
 (gr_line (start 167.3811 121.2186) (end 167.9111 119.9186) (stroke (width 0.153) (type solid)) (layer "Edge.Cuts"))
 (gr_line (start 167.5411 100.4386) (end 166.4811 95.2386) (stroke (width 0.153) (type solid)) (layer "Edge.Cuts"))
 (gr_line (start 167.9111 119.9186) (end 168.3511 118.8086) (stroke (width 0.153) (type solid)) (layer "Edge.Cuts"))
 (gr_line (start 168.3511 105.6786) (end 167.5411 100.4386) (stroke (width 0.153) (type solid)) (layer "Edge.Cuts"))
 (gr_line (start 168.3511 118.8086) (end 168.7011 117.8886) (stroke (width 0.153) (type solid)) (layer "Edge.Cuts"))
 (gr_line (start 168.7011 117.8886) (end 168.9011 117.3186) (stroke (width 0.153) (type solid)) (layer "Edge.Cuts"))
 (gr_line (start 168.9011 117.3186) (end 169.0511 116.8586) (stroke (width 0.153) (type solid)) (layer "Edge.Cuts"))
 (gr_line (start 168.9111 110.9486) (end 168.3511 105.6786) (stroke (width 0.153) (type solid)) (layer "Edge.Cuts"))
 (gr_line (start 168.9711 111.6286) (end 168.9111 110.9486) (stroke (width 0.153) (type solid)) (layer "Edge.Cuts"))
 (gr_line (start 169.0211 112.2686) (end 168.9711 111.6286) (stroke (width 0.153) (type solid)) (layer "Edge.Cuts"))
 (gr_line (start 169.0511 116.8586) (end 169.1811 116.3886) (stroke (width 0.153) (type solid)) (layer "Edge.Cuts"))
 (gr_line (start 169.0611 112.8586) (end 169.0211 112.2686) (stroke (width 0.153) (type solid)) (layer "Edge.Cuts"))
 (gr_line (start 169.1011 113.4086) (end 169.0611 112.8586) (stroke (width 0.153) (type solid)) (layer "Edge.Cuts"))
 (gr_line (start 169.1411 113.9086) (end 169.1011 113.4086) (stroke (width 0.153) (type solid)) (layer "Edge.Cuts"))
 (gr_line (start 169.1611 114.3686) (end 169.1411 113.9086) (stroke (width 0.153) (type solid)) (layer "Edge.Cuts"))
 (gr_line (start 169.1811 116.3886) (end 169.2111 116.0486) (stroke (width 0.153) (type solid)) (layer "Edge.Cuts"))
 (gr_line (start 169.1911 114.7786) (end 169.1611 114.3686) (stroke (width 0.153) (type solid)) (layer "Edge.Cuts"))
 (gr_line (start 169.2111 115.5286) (end 169.1911 114.7786) (stroke (width 0.153) (type solid)) (layer "Edge.Cuts"))
 (gr_line (start 169.2111 116.0486) (end 169.2111 115.5286) (stroke (width 0.153) (type solid)) (layer "Edge.Cuts"))
 (via (at 147.2301 129.2526) (size 1.9304) (drill 1) (layers "F.Cu" "B.Cu") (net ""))
 (via (at 165.4 103.8526) (size 1.9304) (drill 1) (layers "F.Cu" "B.Cu") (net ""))
 (via (at 157.3901 129.2526) (size 1.9304) (drill 1) (layers "F.Cu" "B.Cu") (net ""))
 (via (at 165.4 108.9326) (size 1.9304) (drill 1) (layers "F.Cu" "B.Cu") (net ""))
 (via (at 144.6901 129.2526) (size 1.9304) (drill 1) (layers "F.Cu" "B.Cu") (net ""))
 (via (at 147.2301 116.5526) (size 1.9304) (drill 1) (layers "F.Cu" "B.Cu") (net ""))
 (via (at 152.3101 129.2526) (size 1.9304) (drill 1) (layers "F.Cu" "B.Cu") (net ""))
 (via (at 149.7701 129.2526) (size 1.9304) (drill 1) (layers "F.Cu" "B.Cu") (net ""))
 (via (at 159.9301 131.7926) (size 1.9304) (drill 1) (layers "F.Cu" "B.Cu") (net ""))
 (via (at 149.7701 124.1726) (size 1.9304) (drill 1) (layers "F.Cu" "B.Cu") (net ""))
 (via (at 154.8501 126.7126) (size 1.9304) (drill 1) (layers "F.Cu" "B.Cu") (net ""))
 (via (at 149.7701 121.6326) (size 1.9304) (drill 1) (layers "F.Cu" "B.Cu") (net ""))
 (via (at 159.9301 121.6326) (size 1.9304) (drill 1) (layers "F.Cu" "B.Cu") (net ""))
 (via (at 152.3101 119.0926) (size 1.9304) (drill 1) (layers "F.Cu" "B.Cu") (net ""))
 (via (at 152.3101 121.6326) (size 1.9304) (drill 1) (layers "F.Cu" "B.Cu") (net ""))
 (via (at 159.9301 124.1726) (size 1.9304) (drill 1) (layers "F.Cu" "B.Cu") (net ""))
 (via (at 147.2301 131.7926) (size 1.9304) (drill 1) (layers "F.Cu" "B.Cu") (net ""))
 (via (at 147.2301 126.7126) (size 1.9304) (drill 1) (layers "F.Cu" "B.Cu") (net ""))
 (via (at 159.9301 119.0926) (size 1.9304) (drill 1) (layers "F.Cu" "B.Cu") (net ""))
 (via (at 149.7701 119.0926) (size 1.9304) (drill 1) (layers "F.Cu" "B.Cu") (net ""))
 (via (at 144.6901 126.7126) (size 1.9304) (drill 1) (layers "F.Cu" "B.Cu") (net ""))
 (via (at 159.9301 129.2526) (size 1.9304) (drill 1) (layers "F.Cu" "B.Cu") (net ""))
 (via (at 152.3101 131.7926) (size 1.9304) (drill 1) (layers "F.Cu" "B.Cu") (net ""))
 (via (at 144.6901 131.7926) (size 1.9304) (drill 1) (layers "F.Cu" "B.Cu") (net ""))
 (via (at 157.3901 116.5526) (size 1.9304) (drill 1) (layers "F.Cu" "B.Cu") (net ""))
 (via (at 165.4 98.7726) (size 1.9304) (drill 1) (layers "F.Cu" "B.Cu") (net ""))
 (via (at 152.3101 126.7126) (size 1.9304) (drill 1) (layers "F.Cu" "B.Cu") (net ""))
 (via (at 147.2301 121.6326) (size 1.9304) (drill 1) (layers "F.Cu" "B.Cu") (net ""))
 (via (at 152.3101 116.5526) (size 1.9304) (drill 1) (layers "F.Cu" "B.Cu") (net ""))
 (via (at 157.3901 124.1726) (size 1.9304) (drill 1) (layers "F.Cu" "B.Cu") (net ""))
 (via (at 154.8501 121.6326) (size 1.9304) (drill 1) (layers "F.Cu" "B.Cu") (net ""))
 (via (at 149.7701 116.5526) (size 1.9304) (drill 1) (layers "F.Cu" "B.Cu") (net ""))
 (via (at 165.4 101.3126) (size 1.9304) (drill 1) (layers "F.Cu" "B.Cu") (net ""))
 (via (at 154.8501 124.1726) (size 1.9304) (drill 1) (layers "F.Cu" "B.Cu") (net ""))
 (via (at 144.6901 116.5526) (size 1.9304) (drill 1) (layers "F.Cu" "B.Cu") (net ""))
 (via (at 157.3901 119.0926) (size 1.9304) (drill 1) (layers "F.Cu" "B.Cu") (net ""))
 (via (at 152.3101 124.1726) (size 1.9304) (drill 1) (layers "F.Cu" "B.Cu") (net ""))
 (via (at 157.3901 131.7926) (size 1.9304) (drill 1) (layers "F.Cu" "B.Cu") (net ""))
 (via (at 147.2301 119.0926) (size 1.9304) (drill 1) (layers "F.Cu" "B.Cu") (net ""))
 (via (at 157.3901 121.6326) (size 1.9304) (drill 1) (layers "F.Cu" "B.Cu") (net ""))
 (via (at 147.2301 124.1726) (size 1.9304) (drill 1) (layers "F.Cu" "B.Cu") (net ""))
 (via (at 154.8501 129.2526) (size 1.9304) (drill 1) (layers "F.Cu" "B.Cu") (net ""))
 (via (at 165.4 106.3926) (size 1.9304) (drill 1) (layers "F.Cu" "B.Cu") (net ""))
 (via (at 154.8501 131.7926) (size 1.9304) (drill 1) (layers "F.Cu" "B.Cu") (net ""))
 (via (at 157.3901 126.7126) (size 1.9304) (drill 1) (layers "F.Cu" "B.Cu") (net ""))
 (via (at 154.8501 119.0926) (size 1.9304) (drill 1) (layers "F.Cu" "B.Cu") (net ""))
 (via (at 144.6901 124.1726) (size 1.9304) (drill 1) (layers "F.Cu" "B.Cu") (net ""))
 (via (at 144.6901 119.0926) (size 1.9304) (drill 1) (layers "F.Cu" "B.Cu") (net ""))
 (via (at 162.8701 108.9326) (size 1.9304) (drill 1) (layers "F.Cu" "B.Cu") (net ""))
 (via (at 144.6901 121.6326) (size 1.9304) (drill 1) (layers "F.Cu" "B.Cu") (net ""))
 (via (at 159.9301 126.7126) (size 1.9304) (drill 1) (layers "F.Cu" "B.Cu") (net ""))
 (via (at 149.7701 131.7926) (size 1.9304) (drill 1) (layers "F.Cu" "B.Cu") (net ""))
 (via (at 149.7701 126.7126) (size 1.9304) (drill 1) (layers "F.Cu" "B.Cu") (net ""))
 (via (at 154.8501 116.5526) (size 1.9304) (drill 1) (layers "F.Cu" "B.Cu") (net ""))
 (segment (start 138.3401 124.6726) (end 138.3401 112.7426) (width 0.6096) (layer "F.Cu") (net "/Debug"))
 (segment (start 149.7701 101.3126) (end 159.9301 101.3126) (width 0.6096) (layer "F.Cu") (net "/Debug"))
 (segment (start 138.3401 112.7426) (end 149.7701 101.3126) (width 0.6096) (layer "F.Cu") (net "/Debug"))
 (via (at 162.8701 101.3126) (size 1.9304) (drill 1) (layers "F.Cu" "B.Cu") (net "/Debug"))
 (segment (start 162.97 101.3) (end 160.03 101.3) (width 0.6096) (layer "B.Cu") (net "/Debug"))
 (segment (start 133.0781 104.9406) (end 135.8001 108.9326) (width 0.6096) (layer "F.Cu") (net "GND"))
 (segment (start 131.6 101.4) (end 131.2 101.4) (width 0.6096) (layer "F.Cu") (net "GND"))
 (segment (start 144.6901 108.9326) (end 154.8501 108.9326) (width 0.6096) (layer "F.Cu") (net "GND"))
 (segment (start 131.2 101.4) (end 130 102.6) (width 0.6096) (layer "F.Cu") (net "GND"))
 (segment (start 140.8801 124.6726) (end 140.8801 112.7426) (width 0.6096) (layer "F.Cu") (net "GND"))
 (segment (start 154.8501 108.9326) (end 159.9301 103.8526) (width 0.6096) (layer "F.Cu") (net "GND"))
 (segment (start 140.8801 112.7426) (end 144.6901 108.9326) (width 0.6096) (layer "F.Cu") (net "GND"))
 (segment (start 135.8001 108.9326) (end 139.6101 108.9326) (width 0.6096) (layer "F.Cu") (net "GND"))
 (segment (start 131.2281 104.9406) (end 133.0781 104.9406) (width 0.6096) (layer "F.Cu") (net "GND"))
 (via (at 130 102.6) (size 1.108) (drill 0.6) (layers "F.Cu" "B.Cu") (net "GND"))
 (via (at 139.6101 108.9326) (size 1.108) (drill 0.6) (layers "F.Cu" "B.Cu") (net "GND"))
 (via (at 144.6901 108.9326) (size 1.108) (drill 0.6) (layers "F.Cu" "B.Cu") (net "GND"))
 (via (at 162.8701 103.8526) (size 1.9304) (drill 1) (layers "F.Cu" "B.Cu") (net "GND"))
 (segment (start 162.87 103.9) (end 159.93 103.9) (width 0.6096) (layer "B.Cu") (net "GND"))
 (segment (start 130 103.7125) (end 131.2281 104.9406) (width 0.6096) (layer "B.Cu") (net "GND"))
 (segment (start 130 102.6) (end 130 103.7125) (width 0.6096) (layer "B.Cu") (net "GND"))
 (segment (start 139.6101 108.9326) (end 144.6901 108.9326) (width 0.6096) (layer "B.Cu") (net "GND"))
 (segment (start 133.6 101.4) (end 133.6 103.7002) (width 0.6096) (layer "F.Cu") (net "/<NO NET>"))
 (segment (start 136.8669 103.7002) (end 133.6 103.7002) (width 0.6096) (layer "F.Cu") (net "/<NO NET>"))
 (segment (start 131.2 106.4) (end 130 106.4) (width 0.6096) (layer "F.Cu") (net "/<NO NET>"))
 (segment (start 130 106.4) (end 129.5 105.9) (width 0.6096) (layer "F.Cu") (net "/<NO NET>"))
 (segment (start 130.9233 106.291) (end 131.2281 106.291) (width 0.6096) (layer "F.Cu") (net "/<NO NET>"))
 (segment (start 131.2281 106.291) (end 131.2281 106.4406) (width 0.6096) (layer "F.Cu") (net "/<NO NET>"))
 (segment (start 137.0193 103.8526) (end 137.0701 103.8526) (width 0.6096) (layer "F.Cu") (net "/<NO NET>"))
 (segment (start 133.6 103.7002) (end 130.7709 103.7002) (width 0.6096) (layer "F.Cu") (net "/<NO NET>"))
 (segment (start 130.2998 103.7002) (end 130.7709 103.7002) (width 0.6096) (layer "F.Cu") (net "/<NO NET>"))
 (segment (start 129.5 105.9) (end 129.5 104.5) (width 0.6096) (layer "F.Cu") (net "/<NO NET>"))
 (segment (start 137.0193 103.8526) (end 136.8669 103.7002) (width 0.6096) (layer "F.Cu") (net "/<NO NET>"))
 (segment (start 129.5 104.5) (end 130.2998 103.7002) (width 0.6096) (layer "F.Cu") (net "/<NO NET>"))
 (segment (start 134.16 88.6) (end 134.1 88.66) (width 0.2) (layer "F.Cu") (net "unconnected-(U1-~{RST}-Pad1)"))
 (via (at 134.1 88.66) (size 1.9304) (drill 1) (layers "F.Cu" "B.Cu") (free yes) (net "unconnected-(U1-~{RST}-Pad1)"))
 (segment (start 137.1 88.6) (end 134.16 88.6) (width 0.6096) (layer "B.Cu") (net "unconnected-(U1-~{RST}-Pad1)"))
 (via (at 134.1 91.2) (size 1.9304) (drill 1) (layers "F.Cu" "B.Cu") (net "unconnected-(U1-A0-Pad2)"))
 (segment (start 137.17 91.2) (end 134.23 91.2) (width 0.6096) (layer "B.Cu") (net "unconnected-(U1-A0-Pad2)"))
 (via (at 134.1 93.74) (size 1.9304) (drill 1) (layers "F.Cu" "B.Cu") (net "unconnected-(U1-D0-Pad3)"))
 (segment (start 137.07 93.7) (end 134.13 93.7) (width 0.6096) (layer "B.Cu") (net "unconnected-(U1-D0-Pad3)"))
 (via (at 134.1 96.28) (size 1.9304) (drill 1) (layers "F.Cu" "B.Cu") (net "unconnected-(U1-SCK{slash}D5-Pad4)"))
 (segment (start 137.07 96.3) (end 134.13 96.3) (width 0.6096) (layer "B.Cu") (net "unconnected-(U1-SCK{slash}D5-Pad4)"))
 (via (at 134.1 98.82) (size 1.9304) (drill 1) (layers "F.Cu" "B.Cu") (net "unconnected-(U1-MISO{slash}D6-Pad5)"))
 (segment (start 137.07 98.8) (end 134.13 98.8) (width 0.6096) (layer "B.Cu") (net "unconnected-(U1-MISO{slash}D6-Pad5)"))
 (segment (start 131.2281 107.9406) (end 132.9821 107.9406) (width 0.6096) (layer "B.Cu") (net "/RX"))
 (segment (start 132.9821 107.9406) (end 134.5301 106.3926) (width 0.6096) (layer "B.Cu") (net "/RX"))
 (segment (start 134.5301 103.8526) (end 137.0701 101.3126) (width 0.6096) (layer "B.Cu") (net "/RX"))
 (segment (start 134.5301 106.3926) (end 134.5301 103.8526) (width 0.6096) (layer "B.Cu") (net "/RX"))
 (via (at 162.8701 106.3926) (size 1.9304) (drill 1) (layers "F.Cu" "B.Cu") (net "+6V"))
 (segment (start 133.2601 110.2026) (end 156.1201 110.2026) (width 0.6096) (layer "B.Cu") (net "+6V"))
 (segment (start 162.87 106.4) (end 159.93 106.4) (width 0.6096) (layer "B.Cu") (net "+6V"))
 (segment (start 131.2281 109.4406) (end 132.4981 109.4406) (width 0.6096) (layer "B.Cu") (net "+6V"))
 (segment (start 156.1201 110.2026) (end 159.9301 106.3926) (width 0.6096) (layer "B.Cu") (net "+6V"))
 (segment (start 132.4981 109.4406) (end 133.2601 110.2026) (width 0.6096) (layer "B.Cu") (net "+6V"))
 (via (at 162.8701 98.7726) (size 1.9304) (drill 1) (layers "F.Cu" "B.Cu") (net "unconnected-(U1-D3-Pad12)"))
 (segment (start 162.97 98.8) (end 160.03 98.8) (width 0.6096) (layer "B.Cu") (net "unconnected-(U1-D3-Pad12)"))
 (via (at 162.8701 96.2326) (size 1.9304) (drill 1) (layers "F.Cu" "B.Cu") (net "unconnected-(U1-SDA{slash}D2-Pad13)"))
 (segment (start 162.87 96.2) (end 159.93 96.2) (width 0.6096) (layer "B.Cu") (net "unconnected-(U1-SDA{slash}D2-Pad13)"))
 (via (at 162.8701 93.6926) (size 1.9304) (drill 1) (layers "F.Cu" "B.Cu") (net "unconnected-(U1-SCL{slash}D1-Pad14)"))
 (segment (start 162.97 93.7) (end 160.03 93.7) (width 0.6096) (layer "B.Cu") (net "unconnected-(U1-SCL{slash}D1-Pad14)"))
 (via (at 162.8701 91.1526) (size 1.9304) (drill 1) (layers "F.Cu" "B.Cu") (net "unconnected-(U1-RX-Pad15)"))
 (segment (start 162.87 91.1) (end 159.93 91.1) (width 0.6096) (layer "B.Cu") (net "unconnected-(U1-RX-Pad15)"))
 (via (at 162.8701 88.6126) (size 1.9304) (drill 1) (layers "F.Cu" "B.Cu") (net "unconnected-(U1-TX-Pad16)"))
 (segment (start 162.87 88.6) (end 159.93 88.6) (width 0.6096) (layer "B.Cu") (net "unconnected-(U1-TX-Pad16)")))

